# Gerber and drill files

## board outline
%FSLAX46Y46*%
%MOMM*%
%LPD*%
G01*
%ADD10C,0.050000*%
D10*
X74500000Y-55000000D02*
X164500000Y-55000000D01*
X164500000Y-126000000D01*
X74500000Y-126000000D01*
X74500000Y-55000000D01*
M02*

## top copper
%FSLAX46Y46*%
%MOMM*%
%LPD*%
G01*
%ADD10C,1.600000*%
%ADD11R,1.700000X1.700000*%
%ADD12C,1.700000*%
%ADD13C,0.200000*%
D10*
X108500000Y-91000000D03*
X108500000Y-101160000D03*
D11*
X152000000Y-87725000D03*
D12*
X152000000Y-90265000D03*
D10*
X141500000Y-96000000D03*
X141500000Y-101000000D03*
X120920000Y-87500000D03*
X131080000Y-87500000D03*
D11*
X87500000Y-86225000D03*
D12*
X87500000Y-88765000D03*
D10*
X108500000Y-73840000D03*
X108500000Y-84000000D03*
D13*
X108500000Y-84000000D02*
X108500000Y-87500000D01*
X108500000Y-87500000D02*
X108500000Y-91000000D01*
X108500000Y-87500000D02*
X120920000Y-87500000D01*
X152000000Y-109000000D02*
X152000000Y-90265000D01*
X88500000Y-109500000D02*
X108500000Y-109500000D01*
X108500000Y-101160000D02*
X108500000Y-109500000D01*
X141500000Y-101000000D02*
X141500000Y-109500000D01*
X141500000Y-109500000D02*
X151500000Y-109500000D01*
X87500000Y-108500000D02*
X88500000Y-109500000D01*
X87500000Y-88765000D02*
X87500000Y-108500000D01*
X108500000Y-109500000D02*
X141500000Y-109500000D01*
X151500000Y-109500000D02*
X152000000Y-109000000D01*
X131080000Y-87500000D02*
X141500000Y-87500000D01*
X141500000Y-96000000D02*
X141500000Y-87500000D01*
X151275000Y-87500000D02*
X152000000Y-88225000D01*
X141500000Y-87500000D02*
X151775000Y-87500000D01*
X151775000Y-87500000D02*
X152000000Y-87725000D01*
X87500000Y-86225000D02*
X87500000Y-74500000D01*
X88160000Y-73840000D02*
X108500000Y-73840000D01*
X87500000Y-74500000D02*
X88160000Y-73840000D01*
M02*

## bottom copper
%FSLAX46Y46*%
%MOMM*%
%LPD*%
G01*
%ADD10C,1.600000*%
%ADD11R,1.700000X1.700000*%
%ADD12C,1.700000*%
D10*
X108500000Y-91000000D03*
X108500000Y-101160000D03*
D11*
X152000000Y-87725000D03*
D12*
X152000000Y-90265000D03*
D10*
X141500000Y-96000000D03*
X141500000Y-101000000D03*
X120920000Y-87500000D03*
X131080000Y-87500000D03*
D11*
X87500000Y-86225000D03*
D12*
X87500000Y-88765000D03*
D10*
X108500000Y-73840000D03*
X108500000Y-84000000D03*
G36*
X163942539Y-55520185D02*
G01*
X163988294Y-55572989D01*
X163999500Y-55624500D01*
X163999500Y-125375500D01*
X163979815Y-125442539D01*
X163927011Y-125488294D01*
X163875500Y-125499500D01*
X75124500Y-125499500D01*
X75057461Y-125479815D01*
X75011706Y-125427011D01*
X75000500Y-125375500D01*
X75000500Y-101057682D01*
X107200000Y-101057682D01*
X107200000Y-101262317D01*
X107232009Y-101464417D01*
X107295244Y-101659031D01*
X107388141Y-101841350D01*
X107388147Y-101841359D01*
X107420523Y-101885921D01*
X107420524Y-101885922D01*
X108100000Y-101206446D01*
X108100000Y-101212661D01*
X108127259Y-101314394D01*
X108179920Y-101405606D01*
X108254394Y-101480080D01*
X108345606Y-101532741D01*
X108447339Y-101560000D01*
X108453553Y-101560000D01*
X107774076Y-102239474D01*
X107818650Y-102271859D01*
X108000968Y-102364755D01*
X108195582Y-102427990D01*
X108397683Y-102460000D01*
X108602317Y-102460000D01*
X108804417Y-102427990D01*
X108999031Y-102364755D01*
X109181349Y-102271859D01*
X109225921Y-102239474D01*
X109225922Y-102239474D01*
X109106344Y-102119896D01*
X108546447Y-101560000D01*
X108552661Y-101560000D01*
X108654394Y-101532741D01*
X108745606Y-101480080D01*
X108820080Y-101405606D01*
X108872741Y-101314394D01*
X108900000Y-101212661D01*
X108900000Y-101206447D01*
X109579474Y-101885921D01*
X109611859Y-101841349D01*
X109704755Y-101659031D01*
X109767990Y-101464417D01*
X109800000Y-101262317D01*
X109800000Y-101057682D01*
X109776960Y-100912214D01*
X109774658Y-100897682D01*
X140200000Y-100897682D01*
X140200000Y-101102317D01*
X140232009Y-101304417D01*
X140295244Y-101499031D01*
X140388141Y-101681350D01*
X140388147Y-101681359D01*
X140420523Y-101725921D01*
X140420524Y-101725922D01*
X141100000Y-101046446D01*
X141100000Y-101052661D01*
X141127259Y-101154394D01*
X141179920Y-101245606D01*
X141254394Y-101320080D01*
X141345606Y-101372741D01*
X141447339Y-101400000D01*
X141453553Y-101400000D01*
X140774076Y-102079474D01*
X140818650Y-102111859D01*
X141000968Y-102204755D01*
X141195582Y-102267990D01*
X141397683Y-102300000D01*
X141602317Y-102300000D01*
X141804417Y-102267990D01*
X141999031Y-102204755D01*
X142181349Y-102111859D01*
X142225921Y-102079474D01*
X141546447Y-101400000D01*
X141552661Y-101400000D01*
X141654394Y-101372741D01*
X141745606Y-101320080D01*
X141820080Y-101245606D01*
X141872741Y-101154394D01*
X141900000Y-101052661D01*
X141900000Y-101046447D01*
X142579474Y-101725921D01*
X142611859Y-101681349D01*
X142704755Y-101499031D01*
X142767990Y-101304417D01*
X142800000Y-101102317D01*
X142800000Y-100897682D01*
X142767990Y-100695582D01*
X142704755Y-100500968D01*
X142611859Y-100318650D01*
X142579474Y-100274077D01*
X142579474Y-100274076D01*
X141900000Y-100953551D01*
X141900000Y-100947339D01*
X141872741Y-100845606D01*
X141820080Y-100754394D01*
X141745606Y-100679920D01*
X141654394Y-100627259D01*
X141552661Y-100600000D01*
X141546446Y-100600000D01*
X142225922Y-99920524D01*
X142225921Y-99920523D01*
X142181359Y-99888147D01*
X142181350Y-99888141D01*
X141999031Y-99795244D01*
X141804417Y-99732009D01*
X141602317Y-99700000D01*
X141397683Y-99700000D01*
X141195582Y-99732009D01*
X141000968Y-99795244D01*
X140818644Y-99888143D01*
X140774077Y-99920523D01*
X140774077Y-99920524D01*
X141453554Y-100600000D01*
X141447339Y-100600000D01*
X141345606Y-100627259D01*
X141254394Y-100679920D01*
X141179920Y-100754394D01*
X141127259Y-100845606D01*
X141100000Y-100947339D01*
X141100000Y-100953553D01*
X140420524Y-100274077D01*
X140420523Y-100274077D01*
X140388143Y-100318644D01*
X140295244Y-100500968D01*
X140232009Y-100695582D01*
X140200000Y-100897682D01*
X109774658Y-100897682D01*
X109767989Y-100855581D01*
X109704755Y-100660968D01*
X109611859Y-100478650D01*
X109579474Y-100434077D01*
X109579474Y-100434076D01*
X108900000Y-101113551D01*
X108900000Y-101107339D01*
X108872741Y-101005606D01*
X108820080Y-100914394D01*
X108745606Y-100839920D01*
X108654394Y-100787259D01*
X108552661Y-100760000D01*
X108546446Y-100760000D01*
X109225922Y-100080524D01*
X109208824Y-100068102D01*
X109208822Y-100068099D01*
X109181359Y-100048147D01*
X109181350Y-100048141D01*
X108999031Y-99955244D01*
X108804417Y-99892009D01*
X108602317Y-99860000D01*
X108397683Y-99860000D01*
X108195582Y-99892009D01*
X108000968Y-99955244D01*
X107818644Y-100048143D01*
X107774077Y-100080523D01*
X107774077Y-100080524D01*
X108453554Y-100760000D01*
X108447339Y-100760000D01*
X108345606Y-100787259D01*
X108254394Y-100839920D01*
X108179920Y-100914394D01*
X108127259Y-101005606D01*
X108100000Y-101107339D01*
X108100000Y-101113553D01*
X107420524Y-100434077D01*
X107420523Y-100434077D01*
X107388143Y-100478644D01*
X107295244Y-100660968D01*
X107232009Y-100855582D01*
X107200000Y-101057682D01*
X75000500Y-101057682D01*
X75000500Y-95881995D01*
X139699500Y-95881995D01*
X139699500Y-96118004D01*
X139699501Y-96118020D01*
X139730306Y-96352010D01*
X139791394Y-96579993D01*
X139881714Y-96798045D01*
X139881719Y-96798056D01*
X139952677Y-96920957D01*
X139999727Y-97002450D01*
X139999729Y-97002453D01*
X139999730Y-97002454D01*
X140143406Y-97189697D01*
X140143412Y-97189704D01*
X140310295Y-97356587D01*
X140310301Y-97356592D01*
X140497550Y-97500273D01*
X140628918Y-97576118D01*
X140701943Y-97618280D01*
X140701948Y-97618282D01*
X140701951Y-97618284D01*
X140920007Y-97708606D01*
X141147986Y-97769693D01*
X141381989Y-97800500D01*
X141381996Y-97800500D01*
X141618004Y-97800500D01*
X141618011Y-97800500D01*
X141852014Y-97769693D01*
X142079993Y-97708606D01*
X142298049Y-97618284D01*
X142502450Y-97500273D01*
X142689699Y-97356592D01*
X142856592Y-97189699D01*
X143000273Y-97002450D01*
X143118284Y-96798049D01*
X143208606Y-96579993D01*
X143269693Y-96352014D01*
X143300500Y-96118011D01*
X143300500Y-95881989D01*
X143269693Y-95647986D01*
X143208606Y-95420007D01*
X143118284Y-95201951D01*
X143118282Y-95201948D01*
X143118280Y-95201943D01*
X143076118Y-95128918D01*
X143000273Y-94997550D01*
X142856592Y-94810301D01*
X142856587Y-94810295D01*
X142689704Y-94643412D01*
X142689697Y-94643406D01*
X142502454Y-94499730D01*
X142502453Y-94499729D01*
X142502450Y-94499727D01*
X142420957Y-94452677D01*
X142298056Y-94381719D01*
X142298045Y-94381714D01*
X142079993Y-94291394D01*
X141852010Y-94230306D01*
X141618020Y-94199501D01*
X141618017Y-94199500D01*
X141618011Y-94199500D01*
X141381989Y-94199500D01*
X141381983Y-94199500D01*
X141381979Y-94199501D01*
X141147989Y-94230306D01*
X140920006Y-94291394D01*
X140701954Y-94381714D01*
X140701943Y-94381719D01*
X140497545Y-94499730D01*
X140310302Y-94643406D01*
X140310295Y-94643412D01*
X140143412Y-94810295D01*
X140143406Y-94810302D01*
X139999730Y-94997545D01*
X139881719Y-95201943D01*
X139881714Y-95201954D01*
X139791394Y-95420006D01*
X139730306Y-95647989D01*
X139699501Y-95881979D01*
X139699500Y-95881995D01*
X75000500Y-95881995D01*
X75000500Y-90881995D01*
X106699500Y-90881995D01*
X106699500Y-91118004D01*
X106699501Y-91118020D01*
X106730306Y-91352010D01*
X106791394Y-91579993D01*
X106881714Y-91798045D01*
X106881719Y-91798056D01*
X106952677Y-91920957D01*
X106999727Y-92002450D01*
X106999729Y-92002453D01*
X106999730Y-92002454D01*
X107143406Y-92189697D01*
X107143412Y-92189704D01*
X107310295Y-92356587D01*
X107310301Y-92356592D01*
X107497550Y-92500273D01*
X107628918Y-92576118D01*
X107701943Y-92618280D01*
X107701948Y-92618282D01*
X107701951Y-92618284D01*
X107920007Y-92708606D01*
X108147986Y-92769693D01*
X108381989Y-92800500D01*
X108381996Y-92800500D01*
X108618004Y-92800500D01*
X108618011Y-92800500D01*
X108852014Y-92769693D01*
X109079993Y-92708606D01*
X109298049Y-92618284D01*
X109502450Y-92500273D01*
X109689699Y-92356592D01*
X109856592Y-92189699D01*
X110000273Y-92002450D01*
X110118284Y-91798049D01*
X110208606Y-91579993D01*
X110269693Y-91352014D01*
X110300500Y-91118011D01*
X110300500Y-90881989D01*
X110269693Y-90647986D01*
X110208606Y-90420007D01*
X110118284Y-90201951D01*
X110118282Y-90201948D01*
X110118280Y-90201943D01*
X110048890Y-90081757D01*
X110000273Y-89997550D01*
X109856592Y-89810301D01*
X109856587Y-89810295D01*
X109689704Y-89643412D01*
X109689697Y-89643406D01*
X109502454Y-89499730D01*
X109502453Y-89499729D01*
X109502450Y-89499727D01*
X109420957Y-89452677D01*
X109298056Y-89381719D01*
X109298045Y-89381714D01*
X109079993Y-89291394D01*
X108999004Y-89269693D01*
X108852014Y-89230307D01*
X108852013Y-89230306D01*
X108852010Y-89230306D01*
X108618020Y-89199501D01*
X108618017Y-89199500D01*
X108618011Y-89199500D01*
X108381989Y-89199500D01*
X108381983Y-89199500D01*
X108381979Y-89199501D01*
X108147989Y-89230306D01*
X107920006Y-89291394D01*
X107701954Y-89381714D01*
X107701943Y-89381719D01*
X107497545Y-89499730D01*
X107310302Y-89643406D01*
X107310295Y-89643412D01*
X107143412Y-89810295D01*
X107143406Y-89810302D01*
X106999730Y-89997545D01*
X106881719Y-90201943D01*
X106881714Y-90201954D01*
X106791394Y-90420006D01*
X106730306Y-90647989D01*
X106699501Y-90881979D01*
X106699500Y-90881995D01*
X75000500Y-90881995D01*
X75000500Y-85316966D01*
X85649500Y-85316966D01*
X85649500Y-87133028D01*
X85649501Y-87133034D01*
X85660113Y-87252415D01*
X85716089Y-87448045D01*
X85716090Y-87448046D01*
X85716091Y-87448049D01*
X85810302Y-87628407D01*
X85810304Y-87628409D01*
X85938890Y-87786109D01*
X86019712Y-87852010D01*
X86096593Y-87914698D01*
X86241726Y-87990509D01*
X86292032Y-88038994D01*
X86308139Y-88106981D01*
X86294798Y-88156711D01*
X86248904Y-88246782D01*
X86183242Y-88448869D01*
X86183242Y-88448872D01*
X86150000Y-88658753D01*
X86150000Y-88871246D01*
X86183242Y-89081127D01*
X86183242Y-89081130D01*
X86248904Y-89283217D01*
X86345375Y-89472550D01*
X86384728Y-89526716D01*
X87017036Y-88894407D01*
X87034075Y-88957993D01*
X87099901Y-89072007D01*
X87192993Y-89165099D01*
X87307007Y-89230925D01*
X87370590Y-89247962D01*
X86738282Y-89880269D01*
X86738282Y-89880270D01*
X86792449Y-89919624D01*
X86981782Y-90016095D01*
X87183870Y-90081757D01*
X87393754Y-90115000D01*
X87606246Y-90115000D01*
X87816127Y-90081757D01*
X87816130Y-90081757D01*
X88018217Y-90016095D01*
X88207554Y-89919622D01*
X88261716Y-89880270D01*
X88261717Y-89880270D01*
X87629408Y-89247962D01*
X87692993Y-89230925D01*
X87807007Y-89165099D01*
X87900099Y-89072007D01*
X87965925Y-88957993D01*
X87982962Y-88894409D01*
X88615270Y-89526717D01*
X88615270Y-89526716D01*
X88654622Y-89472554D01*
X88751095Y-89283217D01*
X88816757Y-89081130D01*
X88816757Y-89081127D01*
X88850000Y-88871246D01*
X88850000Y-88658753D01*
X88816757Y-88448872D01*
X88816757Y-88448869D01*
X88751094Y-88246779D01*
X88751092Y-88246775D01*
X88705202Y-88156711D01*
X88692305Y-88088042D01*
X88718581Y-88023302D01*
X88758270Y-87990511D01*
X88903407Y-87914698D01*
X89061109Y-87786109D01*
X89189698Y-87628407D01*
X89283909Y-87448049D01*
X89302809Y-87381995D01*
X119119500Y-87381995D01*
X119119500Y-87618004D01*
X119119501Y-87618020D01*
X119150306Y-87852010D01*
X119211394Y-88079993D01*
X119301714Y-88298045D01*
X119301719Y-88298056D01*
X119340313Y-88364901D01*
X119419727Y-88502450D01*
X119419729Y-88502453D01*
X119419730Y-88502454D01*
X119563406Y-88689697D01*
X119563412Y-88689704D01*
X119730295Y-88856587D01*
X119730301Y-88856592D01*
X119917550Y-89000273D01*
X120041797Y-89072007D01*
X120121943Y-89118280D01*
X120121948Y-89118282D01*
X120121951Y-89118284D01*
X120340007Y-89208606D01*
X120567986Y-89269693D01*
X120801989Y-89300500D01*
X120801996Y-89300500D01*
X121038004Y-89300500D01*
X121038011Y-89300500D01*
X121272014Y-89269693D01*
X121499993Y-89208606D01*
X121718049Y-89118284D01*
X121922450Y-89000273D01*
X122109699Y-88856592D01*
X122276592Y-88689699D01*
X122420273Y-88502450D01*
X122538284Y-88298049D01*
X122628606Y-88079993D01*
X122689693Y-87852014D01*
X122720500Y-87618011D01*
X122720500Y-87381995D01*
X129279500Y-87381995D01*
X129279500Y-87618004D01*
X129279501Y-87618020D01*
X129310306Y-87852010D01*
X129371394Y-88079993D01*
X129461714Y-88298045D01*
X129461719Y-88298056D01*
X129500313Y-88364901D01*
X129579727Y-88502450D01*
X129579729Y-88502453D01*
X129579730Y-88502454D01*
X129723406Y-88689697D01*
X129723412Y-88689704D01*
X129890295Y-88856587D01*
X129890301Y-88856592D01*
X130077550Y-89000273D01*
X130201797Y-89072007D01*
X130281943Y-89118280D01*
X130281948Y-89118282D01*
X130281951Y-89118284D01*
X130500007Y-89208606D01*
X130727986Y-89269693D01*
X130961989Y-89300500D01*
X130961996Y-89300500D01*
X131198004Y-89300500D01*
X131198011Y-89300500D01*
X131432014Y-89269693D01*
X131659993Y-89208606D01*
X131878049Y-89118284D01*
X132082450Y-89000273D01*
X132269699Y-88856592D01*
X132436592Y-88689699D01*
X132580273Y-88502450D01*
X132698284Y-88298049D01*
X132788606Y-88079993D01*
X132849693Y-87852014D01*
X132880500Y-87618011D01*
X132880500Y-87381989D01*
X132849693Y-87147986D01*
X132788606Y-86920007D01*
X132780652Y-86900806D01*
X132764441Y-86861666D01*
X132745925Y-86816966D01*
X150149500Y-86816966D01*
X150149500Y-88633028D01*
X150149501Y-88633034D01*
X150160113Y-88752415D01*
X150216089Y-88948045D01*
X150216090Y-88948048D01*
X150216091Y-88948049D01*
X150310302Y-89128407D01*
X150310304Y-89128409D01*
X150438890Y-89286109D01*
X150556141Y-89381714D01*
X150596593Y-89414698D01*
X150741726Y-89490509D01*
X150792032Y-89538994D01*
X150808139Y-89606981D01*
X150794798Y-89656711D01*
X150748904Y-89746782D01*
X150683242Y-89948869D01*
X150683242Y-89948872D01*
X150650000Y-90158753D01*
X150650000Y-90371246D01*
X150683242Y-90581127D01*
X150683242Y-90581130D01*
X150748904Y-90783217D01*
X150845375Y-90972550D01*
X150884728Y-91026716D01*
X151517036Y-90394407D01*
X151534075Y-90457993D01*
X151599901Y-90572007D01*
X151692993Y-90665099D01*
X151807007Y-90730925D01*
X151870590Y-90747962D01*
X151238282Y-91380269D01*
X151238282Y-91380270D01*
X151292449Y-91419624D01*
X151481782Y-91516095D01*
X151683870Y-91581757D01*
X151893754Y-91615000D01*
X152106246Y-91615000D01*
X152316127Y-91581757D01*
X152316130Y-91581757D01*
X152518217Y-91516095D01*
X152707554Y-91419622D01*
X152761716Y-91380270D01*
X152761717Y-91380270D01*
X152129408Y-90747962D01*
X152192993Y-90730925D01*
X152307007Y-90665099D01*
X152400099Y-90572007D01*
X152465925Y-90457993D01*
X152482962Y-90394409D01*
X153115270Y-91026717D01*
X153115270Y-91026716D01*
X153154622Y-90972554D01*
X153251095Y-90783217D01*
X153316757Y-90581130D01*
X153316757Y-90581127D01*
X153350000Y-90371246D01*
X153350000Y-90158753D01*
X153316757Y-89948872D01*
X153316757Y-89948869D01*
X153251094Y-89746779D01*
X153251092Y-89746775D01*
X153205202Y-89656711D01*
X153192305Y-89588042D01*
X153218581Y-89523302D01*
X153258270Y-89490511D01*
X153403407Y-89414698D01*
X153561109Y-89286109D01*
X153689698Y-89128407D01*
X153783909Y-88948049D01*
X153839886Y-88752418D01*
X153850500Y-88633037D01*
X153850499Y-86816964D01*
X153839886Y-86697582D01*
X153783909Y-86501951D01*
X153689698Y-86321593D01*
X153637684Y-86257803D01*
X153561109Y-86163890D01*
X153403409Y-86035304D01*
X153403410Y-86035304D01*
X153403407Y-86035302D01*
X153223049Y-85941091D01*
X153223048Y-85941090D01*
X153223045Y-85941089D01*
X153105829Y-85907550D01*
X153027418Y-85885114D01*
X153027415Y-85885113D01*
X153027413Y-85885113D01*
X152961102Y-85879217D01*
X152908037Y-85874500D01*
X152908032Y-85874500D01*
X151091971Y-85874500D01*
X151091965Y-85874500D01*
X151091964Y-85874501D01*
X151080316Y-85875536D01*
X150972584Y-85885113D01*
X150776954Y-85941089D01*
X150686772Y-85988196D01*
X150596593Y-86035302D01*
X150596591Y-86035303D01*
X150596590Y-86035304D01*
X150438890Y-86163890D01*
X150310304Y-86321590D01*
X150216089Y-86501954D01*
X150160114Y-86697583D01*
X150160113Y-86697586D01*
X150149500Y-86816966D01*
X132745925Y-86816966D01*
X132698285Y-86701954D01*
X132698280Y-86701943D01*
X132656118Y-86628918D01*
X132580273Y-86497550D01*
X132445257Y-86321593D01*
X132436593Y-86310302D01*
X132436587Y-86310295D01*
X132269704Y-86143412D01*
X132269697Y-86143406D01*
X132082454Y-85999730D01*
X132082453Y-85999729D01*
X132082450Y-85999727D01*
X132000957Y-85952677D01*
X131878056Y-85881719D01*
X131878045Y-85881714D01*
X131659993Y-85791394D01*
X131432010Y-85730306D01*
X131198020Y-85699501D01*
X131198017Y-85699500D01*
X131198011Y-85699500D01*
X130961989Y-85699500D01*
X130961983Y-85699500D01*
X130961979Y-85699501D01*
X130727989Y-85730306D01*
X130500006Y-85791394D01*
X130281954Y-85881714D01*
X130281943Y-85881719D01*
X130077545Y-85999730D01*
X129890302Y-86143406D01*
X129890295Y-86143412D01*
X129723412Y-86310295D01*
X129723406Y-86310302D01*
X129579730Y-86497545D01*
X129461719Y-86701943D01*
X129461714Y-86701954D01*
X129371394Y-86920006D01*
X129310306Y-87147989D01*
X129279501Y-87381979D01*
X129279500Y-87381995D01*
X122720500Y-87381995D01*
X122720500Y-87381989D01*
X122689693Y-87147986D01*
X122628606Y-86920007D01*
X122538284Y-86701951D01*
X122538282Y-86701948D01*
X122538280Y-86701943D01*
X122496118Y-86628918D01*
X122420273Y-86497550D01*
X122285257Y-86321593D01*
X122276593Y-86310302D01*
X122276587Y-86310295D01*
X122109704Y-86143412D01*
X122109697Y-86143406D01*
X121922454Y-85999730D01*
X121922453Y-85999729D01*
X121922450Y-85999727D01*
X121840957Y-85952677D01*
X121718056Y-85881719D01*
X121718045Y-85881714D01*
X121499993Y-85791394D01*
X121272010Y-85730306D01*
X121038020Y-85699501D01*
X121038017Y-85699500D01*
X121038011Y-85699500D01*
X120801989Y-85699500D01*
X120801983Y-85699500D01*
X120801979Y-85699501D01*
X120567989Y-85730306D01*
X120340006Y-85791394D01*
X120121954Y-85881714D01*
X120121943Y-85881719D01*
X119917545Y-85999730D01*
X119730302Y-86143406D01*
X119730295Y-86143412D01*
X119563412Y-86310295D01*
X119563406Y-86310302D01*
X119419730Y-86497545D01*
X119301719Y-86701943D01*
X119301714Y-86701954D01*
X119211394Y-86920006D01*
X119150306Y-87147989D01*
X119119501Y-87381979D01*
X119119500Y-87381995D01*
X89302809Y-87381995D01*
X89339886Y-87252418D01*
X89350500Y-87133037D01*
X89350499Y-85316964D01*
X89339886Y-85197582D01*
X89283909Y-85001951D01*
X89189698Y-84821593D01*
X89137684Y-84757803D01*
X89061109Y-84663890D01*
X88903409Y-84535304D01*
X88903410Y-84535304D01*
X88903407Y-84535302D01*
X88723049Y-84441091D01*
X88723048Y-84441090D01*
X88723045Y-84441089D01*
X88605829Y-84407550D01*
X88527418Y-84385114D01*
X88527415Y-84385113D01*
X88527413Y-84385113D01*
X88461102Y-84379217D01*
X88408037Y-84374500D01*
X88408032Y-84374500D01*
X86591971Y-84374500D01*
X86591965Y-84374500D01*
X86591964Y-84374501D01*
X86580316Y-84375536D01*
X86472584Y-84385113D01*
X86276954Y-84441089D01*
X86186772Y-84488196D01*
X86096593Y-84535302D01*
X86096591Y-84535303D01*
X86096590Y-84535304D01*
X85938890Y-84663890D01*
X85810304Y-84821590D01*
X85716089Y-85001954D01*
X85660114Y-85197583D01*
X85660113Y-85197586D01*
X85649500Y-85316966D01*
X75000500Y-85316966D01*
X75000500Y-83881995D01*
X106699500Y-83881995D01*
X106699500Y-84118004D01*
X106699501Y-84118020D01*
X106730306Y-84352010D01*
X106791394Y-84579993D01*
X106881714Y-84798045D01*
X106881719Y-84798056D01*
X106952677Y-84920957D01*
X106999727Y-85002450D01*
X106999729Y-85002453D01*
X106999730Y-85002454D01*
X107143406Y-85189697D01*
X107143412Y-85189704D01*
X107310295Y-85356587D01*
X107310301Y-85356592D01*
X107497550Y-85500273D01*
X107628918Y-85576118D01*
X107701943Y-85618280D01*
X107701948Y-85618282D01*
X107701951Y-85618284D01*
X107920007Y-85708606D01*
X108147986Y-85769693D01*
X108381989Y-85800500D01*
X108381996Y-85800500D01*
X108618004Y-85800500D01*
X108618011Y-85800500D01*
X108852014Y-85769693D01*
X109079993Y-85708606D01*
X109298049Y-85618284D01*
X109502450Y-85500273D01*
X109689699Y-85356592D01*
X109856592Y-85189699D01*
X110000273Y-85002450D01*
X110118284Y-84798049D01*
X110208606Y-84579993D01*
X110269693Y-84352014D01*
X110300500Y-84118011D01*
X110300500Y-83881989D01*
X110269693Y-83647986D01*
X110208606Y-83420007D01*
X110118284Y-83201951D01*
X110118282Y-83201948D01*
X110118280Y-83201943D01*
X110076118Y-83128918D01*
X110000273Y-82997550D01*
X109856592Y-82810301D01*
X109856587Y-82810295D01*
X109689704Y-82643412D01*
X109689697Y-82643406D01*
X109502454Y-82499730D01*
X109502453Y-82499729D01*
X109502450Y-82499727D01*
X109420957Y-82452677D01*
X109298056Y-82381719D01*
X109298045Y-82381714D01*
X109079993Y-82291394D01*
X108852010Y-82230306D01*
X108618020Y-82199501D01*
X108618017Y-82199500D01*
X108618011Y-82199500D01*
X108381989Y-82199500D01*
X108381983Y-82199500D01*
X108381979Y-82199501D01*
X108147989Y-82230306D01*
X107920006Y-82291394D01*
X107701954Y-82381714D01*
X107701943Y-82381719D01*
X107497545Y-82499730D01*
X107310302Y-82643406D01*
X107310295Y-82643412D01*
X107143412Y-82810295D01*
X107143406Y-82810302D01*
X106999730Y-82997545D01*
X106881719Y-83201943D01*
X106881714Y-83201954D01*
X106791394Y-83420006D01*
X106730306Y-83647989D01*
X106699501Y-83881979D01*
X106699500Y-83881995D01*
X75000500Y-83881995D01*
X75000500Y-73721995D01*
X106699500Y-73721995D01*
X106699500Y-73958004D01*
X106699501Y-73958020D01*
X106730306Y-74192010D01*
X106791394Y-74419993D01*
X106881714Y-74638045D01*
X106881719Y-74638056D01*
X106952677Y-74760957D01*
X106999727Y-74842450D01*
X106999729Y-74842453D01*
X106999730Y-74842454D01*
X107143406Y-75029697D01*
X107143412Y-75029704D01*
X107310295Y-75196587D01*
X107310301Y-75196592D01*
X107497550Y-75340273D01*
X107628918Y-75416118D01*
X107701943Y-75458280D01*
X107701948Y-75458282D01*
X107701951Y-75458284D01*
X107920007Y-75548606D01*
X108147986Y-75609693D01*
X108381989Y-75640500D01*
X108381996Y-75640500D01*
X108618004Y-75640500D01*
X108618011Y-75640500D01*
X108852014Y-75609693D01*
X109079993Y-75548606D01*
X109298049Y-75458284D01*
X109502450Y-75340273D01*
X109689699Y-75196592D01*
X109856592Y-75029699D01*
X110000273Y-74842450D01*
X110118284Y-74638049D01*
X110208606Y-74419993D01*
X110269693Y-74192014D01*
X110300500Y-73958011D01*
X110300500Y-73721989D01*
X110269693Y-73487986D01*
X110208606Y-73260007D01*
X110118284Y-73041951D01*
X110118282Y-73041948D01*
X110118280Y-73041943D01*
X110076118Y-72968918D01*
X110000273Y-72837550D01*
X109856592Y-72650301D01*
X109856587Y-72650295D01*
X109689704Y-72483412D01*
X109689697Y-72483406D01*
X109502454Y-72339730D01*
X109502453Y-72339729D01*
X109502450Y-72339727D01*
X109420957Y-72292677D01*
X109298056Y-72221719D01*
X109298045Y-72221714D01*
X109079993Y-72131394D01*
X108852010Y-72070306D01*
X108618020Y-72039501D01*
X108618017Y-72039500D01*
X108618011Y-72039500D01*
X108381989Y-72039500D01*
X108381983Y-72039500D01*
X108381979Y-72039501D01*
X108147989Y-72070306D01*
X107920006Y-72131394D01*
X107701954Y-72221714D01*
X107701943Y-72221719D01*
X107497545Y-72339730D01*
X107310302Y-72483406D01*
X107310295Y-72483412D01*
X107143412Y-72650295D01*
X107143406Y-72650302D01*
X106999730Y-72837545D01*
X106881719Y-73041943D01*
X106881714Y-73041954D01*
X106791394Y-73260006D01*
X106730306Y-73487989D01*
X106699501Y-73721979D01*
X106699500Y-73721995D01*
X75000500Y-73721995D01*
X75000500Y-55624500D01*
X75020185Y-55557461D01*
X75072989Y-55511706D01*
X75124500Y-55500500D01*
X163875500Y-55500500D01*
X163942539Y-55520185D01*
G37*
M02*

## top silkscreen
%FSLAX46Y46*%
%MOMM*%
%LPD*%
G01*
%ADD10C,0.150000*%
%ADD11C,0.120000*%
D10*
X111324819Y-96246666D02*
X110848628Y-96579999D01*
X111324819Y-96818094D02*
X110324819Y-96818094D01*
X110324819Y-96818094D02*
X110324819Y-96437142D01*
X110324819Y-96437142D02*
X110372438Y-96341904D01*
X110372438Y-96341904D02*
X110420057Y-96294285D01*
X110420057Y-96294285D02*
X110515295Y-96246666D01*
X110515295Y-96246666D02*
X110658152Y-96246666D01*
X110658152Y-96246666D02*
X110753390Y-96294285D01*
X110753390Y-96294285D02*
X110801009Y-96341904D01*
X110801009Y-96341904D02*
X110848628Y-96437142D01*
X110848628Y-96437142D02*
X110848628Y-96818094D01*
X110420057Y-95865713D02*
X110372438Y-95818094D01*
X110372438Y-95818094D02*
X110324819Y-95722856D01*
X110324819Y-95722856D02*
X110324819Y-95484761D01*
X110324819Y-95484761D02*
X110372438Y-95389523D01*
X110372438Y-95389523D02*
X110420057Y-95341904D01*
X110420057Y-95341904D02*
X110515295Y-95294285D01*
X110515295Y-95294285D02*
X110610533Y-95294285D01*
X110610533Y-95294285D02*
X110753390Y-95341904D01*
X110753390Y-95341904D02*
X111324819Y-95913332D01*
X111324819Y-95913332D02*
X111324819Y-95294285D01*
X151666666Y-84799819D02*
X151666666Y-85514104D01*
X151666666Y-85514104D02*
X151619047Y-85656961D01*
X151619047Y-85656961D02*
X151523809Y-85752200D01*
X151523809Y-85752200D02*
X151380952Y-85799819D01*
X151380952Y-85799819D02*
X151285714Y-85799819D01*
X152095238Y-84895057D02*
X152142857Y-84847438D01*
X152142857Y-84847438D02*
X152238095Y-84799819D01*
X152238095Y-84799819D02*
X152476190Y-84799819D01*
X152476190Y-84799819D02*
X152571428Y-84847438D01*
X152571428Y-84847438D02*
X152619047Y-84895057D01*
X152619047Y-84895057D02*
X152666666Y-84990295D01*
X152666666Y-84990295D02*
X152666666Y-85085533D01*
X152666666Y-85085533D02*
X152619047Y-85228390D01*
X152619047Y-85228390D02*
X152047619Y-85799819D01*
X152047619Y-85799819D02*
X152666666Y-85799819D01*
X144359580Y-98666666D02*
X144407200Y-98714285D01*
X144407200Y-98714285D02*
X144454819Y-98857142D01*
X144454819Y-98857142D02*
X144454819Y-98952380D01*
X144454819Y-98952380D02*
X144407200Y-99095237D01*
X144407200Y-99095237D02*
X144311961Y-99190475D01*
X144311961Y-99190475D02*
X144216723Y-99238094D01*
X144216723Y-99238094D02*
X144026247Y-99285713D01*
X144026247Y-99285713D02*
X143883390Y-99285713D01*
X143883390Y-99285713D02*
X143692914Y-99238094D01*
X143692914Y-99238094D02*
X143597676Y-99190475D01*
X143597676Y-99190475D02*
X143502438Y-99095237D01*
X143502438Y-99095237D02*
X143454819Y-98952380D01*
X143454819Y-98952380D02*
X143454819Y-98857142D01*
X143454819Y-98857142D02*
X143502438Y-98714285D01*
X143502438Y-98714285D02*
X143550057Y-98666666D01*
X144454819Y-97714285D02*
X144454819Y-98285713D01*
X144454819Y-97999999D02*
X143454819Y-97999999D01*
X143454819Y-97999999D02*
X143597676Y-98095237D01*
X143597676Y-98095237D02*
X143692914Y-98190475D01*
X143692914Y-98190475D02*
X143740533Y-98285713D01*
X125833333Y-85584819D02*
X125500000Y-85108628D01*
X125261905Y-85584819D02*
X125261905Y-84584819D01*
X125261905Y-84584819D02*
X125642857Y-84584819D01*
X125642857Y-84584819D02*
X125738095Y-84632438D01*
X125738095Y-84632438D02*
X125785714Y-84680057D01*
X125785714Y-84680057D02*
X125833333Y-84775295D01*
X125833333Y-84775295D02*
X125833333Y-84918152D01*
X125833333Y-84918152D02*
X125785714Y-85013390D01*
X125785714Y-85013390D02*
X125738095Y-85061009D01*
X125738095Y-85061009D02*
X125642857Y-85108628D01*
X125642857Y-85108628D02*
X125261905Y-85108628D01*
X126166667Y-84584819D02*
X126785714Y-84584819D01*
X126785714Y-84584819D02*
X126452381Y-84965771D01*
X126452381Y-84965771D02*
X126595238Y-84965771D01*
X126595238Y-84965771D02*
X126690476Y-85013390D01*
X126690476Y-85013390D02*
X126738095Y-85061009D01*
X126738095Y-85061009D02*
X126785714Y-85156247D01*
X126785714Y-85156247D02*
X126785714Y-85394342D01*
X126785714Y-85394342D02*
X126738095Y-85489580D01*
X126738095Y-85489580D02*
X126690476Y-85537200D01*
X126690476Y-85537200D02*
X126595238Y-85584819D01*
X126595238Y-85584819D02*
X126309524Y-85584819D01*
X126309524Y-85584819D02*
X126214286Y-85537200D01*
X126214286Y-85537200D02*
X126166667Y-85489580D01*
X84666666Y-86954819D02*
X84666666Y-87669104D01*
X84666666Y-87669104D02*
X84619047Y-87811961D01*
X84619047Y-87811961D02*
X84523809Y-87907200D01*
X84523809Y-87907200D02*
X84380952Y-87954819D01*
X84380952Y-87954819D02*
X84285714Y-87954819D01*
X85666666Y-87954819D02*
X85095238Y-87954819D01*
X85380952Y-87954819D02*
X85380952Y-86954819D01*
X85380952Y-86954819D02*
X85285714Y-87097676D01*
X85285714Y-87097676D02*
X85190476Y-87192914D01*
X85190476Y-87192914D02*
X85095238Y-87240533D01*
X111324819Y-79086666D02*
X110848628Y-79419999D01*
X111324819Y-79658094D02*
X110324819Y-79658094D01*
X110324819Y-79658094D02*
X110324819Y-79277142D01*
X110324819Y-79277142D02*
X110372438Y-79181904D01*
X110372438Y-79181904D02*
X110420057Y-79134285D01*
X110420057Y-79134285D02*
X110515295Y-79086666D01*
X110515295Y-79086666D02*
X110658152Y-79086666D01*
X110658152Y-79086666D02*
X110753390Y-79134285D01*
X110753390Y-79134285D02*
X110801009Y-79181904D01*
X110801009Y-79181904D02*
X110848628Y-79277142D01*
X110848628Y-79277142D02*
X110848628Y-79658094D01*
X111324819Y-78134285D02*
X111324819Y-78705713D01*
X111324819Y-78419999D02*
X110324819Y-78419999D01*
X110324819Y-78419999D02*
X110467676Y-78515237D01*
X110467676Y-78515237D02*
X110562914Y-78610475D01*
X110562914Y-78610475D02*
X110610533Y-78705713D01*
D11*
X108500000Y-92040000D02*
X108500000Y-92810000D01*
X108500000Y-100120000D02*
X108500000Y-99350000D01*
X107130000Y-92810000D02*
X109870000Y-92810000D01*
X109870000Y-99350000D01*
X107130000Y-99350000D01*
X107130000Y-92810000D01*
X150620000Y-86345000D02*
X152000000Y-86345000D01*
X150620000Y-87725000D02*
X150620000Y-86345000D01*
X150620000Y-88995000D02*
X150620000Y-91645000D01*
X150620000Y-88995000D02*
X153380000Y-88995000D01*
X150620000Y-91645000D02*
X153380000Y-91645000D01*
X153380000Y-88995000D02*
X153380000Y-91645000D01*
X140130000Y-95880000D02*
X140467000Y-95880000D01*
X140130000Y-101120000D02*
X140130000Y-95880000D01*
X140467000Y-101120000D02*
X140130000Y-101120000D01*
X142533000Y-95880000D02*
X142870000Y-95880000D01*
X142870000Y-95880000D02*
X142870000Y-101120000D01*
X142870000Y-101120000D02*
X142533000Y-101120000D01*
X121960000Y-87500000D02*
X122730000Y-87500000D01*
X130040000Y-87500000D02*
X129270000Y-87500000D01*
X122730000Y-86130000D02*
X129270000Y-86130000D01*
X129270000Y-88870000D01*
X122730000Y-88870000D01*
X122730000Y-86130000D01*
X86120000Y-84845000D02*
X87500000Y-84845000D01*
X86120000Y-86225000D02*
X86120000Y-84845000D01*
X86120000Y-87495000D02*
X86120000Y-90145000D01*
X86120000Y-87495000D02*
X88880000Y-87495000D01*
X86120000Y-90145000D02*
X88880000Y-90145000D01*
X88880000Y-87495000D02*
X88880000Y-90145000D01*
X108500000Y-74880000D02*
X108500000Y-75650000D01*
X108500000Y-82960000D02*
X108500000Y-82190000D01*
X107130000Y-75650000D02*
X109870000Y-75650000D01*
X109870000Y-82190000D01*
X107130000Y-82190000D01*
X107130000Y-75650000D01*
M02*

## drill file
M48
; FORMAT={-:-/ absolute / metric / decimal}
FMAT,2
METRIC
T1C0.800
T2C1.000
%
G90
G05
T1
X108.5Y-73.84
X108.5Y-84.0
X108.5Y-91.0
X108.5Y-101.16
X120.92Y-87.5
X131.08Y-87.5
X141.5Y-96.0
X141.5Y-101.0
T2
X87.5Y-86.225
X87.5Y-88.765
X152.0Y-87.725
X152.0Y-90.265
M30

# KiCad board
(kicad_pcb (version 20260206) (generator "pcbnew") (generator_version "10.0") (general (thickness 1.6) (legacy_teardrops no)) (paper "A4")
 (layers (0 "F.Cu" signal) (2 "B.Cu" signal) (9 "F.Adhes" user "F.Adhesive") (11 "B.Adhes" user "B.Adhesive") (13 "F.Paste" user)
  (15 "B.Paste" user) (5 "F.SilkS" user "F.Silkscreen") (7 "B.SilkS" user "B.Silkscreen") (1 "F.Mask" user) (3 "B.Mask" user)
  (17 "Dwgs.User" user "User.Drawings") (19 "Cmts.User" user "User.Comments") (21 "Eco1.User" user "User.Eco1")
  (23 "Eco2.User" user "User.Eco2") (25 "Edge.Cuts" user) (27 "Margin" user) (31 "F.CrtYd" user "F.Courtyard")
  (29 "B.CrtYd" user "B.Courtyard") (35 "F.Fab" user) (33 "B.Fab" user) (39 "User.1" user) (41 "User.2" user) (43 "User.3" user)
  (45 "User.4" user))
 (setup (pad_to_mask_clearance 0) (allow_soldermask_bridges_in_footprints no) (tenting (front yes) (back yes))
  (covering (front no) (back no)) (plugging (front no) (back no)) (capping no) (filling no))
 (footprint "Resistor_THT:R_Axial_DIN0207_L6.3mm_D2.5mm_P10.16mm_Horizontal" (layer "F.Cu") (at 108.5 91 -90)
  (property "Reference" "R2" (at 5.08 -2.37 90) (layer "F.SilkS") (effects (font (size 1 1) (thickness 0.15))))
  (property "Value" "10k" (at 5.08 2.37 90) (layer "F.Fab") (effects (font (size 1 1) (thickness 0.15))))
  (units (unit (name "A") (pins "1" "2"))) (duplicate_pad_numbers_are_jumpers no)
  (fp_line (start 1.04 0) (end 1.81 0) (stroke (width 0.12) (type solid)) (layer "F.SilkS"))
  (fp_line (start 9.12 0) (end 8.35 0) (stroke (width 0.12) (type solid)) (layer "F.SilkS"))
  (fp_rect (start 1.81 -1.37) (end 8.35 1.37) (stroke (width 0.12) (type solid)) (fill no) (layer "F.SilkS"))
  (pad "1" thru_hole circle (at 0 0 270) (size 1.6 1.6) (drill 0.8) (layers "*.Cu" "*.Mask") (remove_unused_layers no) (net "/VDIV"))
  (pad "2" thru_hole circle (at 10.16 0 270) (size 1.6 1.6) (drill 0.8) (layers "*.Cu" "*.Mask") (remove_unused_layers no) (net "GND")))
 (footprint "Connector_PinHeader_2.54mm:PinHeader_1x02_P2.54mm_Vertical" (layer "F.Cu") (at 152 87.725)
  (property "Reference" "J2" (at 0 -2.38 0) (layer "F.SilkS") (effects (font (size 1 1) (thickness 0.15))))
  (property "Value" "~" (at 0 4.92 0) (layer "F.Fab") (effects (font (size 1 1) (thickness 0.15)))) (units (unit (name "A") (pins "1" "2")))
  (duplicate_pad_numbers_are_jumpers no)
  (fp_line (start -1.38 -1.38) (end 0 -1.38) (stroke (width 0.12) (type solid)) (layer "F.SilkS"))
  (fp_line (start -1.38 0) (end -1.38 -1.38) (stroke (width 0.12) (type solid)) (layer "F.SilkS"))
  (fp_line (start -1.38 1.27) (end -1.38 3.92) (stroke (width 0.12) (type solid)) (layer "F.SilkS"))
  (fp_line (start -1.38 1.27) (end 1.38 1.27) (stroke (width 0.12) (type solid)) (layer "F.SilkS"))
  (fp_line (start -1.38 3.92) (end 1.38 3.92) (stroke (width 0.12) (type solid)) (layer "F.SilkS"))
  (fp_line (start 1.38 1.27) (end 1.38 3.92) (stroke (width 0.12) (type solid)) (layer "F.SilkS"))
  (pad "1" thru_hole rect (at 0 0) (size 1.7 1.7) (drill 1) (layers "*.Cu" "*.Mask") (remove_unused_layers no) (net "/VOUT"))
  (pad "2" thru_hole circle (at 0 2.54) (size 1.7 1.7) (drill 1) (layers "*.Cu" "*.Mask") (remove_unused_layers no) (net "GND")))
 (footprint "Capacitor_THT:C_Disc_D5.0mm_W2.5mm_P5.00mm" (layer "F.Cu") (at 141.5 96 -90)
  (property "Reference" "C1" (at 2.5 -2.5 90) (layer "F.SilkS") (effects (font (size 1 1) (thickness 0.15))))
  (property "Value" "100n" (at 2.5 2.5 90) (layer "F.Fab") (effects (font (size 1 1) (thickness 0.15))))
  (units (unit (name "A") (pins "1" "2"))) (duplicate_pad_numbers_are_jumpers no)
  (fp_line (start -0.12 1.37) (end -0.12 1.033) (stroke (width 0.12) (type solid)) (layer "F.SilkS"))
  (fp_line (start 5.12 1.37) (end -0.12 1.37) (stroke (width 0.12) (type solid)) (layer "F.SilkS"))
  (fp_line (start 5.12 1.033) (end 5.12 1.37) (stroke (width 0.12) (type solid)) (layer "F.SilkS"))
  (fp_line (start -0.12 -1.033) (end -0.12 -1.37) (stroke (width 0.12) (type solid)) (layer "F.SilkS"))
  (fp_line (start -0.12 -1.37) (end 5.12 -1.37) (stroke (width 0.12) (type solid)) (layer "F.SilkS"))
  (fp_line (start 5.12 -1.37) (end 5.12 -1.033) (stroke (width 0.12) (type solid)) (layer "F.SilkS"))
  (pad "1" thru_hole circle (at 0 0 270) (size 1.6 1.6) (drill 0.8) (layers "*.Cu" "*.Mask") (remove_unused_layers no) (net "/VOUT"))
  (pad "2" thru_hole circle (at 5 0 270) (size 1.6 1.6) (drill 0.8) (layers "*.Cu" "*.Mask") (remove_unused_layers no) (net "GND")))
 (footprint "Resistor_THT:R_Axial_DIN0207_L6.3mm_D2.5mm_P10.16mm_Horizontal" (layer "F.Cu") (at 120.92 87.5)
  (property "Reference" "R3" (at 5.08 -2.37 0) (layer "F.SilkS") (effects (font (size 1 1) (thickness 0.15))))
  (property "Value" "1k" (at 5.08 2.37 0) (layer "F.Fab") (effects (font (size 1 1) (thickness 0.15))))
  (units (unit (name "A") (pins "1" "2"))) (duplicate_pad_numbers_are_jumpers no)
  (fp_line (start 1.04 0) (end 1.81 0) (stroke (width 0.12) (type solid)) (layer "F.SilkS"))
  (fp_line (start 9.12 0) (end 8.35 0) (stroke (width 0.12) (type solid)) (layer "F.SilkS"))
  (fp_rect (start 1.81 -1.37) (end 8.35 1.37) (stroke (width 0.12) (type solid)) (fill no) (layer "F.SilkS"))
  (pad "1" thru_hole circle (at 0 0) (size 1.6 1.6) (drill 0.8) (layers "*.Cu" "*.Mask") (remove_unused_layers no) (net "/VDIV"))
  (pad "2" thru_hole circle (at 10.16 0) (size 1.6 1.6) (drill 0.8) (layers "*.Cu" "*.Mask") (remove_unused_layers no) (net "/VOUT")))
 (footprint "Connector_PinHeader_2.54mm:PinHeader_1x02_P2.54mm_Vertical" (layer "F.Cu") (at 87.5 86.225)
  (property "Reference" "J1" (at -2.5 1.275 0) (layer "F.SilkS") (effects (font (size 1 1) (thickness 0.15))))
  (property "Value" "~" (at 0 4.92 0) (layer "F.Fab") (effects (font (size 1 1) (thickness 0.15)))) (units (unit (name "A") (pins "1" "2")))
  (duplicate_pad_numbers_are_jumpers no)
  (fp_line (start -1.38 -1.38) (end 0 -1.38) (stroke (width 0.12) (type solid)) (layer "F.SilkS"))
  (fp_line (start -1.38 0) (end -1.38 -1.38) (stroke (width 0.12) (type solid)) (layer "F.SilkS"))
  (fp_line (start -1.38 1.27) (end -1.38 3.92) (stroke (width 0.12) (type solid)) (layer "F.SilkS"))
  (fp_line (start -1.38 1.27) (end 1.38 1.27) (stroke (width 0.12) (type solid)) (layer "F.SilkS"))
  (fp_line (start -1.38 3.92) (end 1.38 3.92) (stroke (width 0.12) (type solid)) (layer "F.SilkS"))
  (fp_line (start 1.38 1.27) (end 1.38 3.92) (stroke (width 0.12) (type solid)) (layer "F.SilkS"))
  (pad "1" thru_hole rect (at 0 0) (size 1.7 1.7) (drill 1) (layers "*.Cu" "*.Mask") (remove_unused_layers no) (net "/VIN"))
  (pad "2" thru_hole circle (at 0 2.54) (size 1.7 1.7) (drill 1) (layers "*.Cu" "*.Mask") (remove_unused_layers no) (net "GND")))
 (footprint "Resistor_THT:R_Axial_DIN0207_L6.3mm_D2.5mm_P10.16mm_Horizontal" (layer "F.Cu") (at 108.5 73.84 -90)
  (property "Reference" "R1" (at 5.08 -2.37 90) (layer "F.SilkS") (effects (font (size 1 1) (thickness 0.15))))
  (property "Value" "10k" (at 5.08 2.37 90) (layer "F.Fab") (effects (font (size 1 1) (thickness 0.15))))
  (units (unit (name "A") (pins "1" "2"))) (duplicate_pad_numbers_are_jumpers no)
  (fp_line (start 1.04 0) (end 1.81 0) (stroke (width 0.12) (type solid)) (layer "F.SilkS"))
  (fp_line (start 9.12 0) (end 8.35 0) (stroke (width 0.12) (type solid)) (layer "F.SilkS"))
  (fp_rect (start 1.81 -1.37) (end 8.35 1.37) (stroke (width 0.12) (type solid)) (fill no) (layer "F.SilkS"))
  (pad "1" thru_hole circle (at 0 0 270) (size 1.6 1.6) (drill 0.8) (layers "*.Cu" "*.Mask") (remove_unused_layers no) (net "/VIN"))
  (pad "2" thru_hole circle (at 10.16 0 270) (size 1.6 1.6) (drill 0.8) (layers "*.Cu" "*.Mask") (remove_unused_layers no) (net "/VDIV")))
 (gr_rect (start 74.5 55) (end 164.5 126) (stroke (width 0.05) (type default)) (fill no) (layer "Edge.Cuts"))
 (segment (start 108.5 84) (end 108.5 87.5) (width 0.2) (layers "F.Cu" "F.Mask") (solder_mask_margin 0.2) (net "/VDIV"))
 (segment (start 108.5 87.5) (end 108.5 91) (width 0.2) (layers "F.Cu" "F.Mask") (solder_mask_margin 0.2) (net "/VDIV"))
 (segment (start 108.5 87.5) (end 120.92 87.5) (width 0.2) (layers "F.Cu" "F.Mask") (solder_mask_margin 0.2) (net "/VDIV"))
 (segment (start 152 109) (end 152 90.265) (width 0.2) (layers "F.Cu" "F.Mask") (solder_mask_margin 0.2) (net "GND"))
 (segment (start 88.5 109.5) (end 108.5 109.5) (width 0.2) (layers "F.Cu" "F.Mask") (solder_mask_margin 0.2) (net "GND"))
 (segment (start 108.5 101.16) (end 108.5 109.5) (width 0.2) (layers "F.Cu" "F.Mask") (solder_mask_margin 0.2) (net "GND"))
 (segment (start 141.5 101) (end 141.5 109.5) (width 0.2) (layers "F.Cu" "F.Mask") (solder_mask_margin 0.2) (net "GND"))
 (segment (start 141.5 109.5) (end 151.5 109.5) (width 0.2) (layers "F.Cu" "F.Mask") (solder_mask_margin 0.2) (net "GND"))
 (segment (start 87.5 108.5) (end 88.5 109.5) (width 0.2) (layers "F.Cu" "F.Mask") (solder_mask_margin 0.2) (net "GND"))
 (segment (start 87.5 88.765) (end 87.5 108.5) (width 0.2) (layers "F.Cu" "F.Mask") (solder_mask_margin 0.2) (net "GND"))
 (segment (start 108.5 109.5) (end 141.5 109.5) (width 0.2) (layers "F.Cu" "F.Mask") (solder_mask_margin 0.2) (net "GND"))
 (segment (start 151.5 109.5) (end 152 109) (width 0.2) (layers "F.Cu" "F.Mask") (solder_mask_margin 0.2) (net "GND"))
 (segment (start 131.08 87.5) (end 141.5 87.5) (width 0.2) (layers "F.Cu" "F.Mask") (solder_mask_margin 0.2) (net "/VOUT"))
 (segment (start 141.5 96) (end 141.5 87.5) (width 0.2) (layers "F.Cu" "F.Mask") (solder_mask_margin 0.2) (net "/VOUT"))
 (segment (start 151.275 87.5) (end 152 88.225) (width 0.2) (layer "F.Cu") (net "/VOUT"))
 (segment (start 141.5 87.5) (end 151.775 87.5) (width 0.2) (layers "F.Cu" "F.Mask") (solder_mask_margin 0.2) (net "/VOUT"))
 (segment (start 151.775 87.5) (end 152 87.725) (width 0.2) (layers "F.Cu" "F.Mask") (solder_mask_margin 0.2) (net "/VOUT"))
 (segment (start 87.5 86.225) (end 87.5 74.5) (width 0.2) (layers "F.Cu" "F.Mask") (solder_mask_margin 0.2) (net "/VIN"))
 (segment (start 88.16 73.84) (end 108.5 73.84) (width 0.2) (layers "F.Cu" "F.Mask") (solder_mask_margin 0.2) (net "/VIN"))
 (segment (start 87.5 74.5) (end 88.16 73.84) (width 0.2) (layers "F.Cu" "F.Mask") (solder_mask_margin 0.2) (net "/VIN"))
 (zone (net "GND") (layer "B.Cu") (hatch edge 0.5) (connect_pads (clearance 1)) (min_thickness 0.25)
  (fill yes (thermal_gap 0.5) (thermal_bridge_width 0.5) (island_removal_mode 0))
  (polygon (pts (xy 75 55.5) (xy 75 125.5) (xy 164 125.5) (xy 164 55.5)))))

